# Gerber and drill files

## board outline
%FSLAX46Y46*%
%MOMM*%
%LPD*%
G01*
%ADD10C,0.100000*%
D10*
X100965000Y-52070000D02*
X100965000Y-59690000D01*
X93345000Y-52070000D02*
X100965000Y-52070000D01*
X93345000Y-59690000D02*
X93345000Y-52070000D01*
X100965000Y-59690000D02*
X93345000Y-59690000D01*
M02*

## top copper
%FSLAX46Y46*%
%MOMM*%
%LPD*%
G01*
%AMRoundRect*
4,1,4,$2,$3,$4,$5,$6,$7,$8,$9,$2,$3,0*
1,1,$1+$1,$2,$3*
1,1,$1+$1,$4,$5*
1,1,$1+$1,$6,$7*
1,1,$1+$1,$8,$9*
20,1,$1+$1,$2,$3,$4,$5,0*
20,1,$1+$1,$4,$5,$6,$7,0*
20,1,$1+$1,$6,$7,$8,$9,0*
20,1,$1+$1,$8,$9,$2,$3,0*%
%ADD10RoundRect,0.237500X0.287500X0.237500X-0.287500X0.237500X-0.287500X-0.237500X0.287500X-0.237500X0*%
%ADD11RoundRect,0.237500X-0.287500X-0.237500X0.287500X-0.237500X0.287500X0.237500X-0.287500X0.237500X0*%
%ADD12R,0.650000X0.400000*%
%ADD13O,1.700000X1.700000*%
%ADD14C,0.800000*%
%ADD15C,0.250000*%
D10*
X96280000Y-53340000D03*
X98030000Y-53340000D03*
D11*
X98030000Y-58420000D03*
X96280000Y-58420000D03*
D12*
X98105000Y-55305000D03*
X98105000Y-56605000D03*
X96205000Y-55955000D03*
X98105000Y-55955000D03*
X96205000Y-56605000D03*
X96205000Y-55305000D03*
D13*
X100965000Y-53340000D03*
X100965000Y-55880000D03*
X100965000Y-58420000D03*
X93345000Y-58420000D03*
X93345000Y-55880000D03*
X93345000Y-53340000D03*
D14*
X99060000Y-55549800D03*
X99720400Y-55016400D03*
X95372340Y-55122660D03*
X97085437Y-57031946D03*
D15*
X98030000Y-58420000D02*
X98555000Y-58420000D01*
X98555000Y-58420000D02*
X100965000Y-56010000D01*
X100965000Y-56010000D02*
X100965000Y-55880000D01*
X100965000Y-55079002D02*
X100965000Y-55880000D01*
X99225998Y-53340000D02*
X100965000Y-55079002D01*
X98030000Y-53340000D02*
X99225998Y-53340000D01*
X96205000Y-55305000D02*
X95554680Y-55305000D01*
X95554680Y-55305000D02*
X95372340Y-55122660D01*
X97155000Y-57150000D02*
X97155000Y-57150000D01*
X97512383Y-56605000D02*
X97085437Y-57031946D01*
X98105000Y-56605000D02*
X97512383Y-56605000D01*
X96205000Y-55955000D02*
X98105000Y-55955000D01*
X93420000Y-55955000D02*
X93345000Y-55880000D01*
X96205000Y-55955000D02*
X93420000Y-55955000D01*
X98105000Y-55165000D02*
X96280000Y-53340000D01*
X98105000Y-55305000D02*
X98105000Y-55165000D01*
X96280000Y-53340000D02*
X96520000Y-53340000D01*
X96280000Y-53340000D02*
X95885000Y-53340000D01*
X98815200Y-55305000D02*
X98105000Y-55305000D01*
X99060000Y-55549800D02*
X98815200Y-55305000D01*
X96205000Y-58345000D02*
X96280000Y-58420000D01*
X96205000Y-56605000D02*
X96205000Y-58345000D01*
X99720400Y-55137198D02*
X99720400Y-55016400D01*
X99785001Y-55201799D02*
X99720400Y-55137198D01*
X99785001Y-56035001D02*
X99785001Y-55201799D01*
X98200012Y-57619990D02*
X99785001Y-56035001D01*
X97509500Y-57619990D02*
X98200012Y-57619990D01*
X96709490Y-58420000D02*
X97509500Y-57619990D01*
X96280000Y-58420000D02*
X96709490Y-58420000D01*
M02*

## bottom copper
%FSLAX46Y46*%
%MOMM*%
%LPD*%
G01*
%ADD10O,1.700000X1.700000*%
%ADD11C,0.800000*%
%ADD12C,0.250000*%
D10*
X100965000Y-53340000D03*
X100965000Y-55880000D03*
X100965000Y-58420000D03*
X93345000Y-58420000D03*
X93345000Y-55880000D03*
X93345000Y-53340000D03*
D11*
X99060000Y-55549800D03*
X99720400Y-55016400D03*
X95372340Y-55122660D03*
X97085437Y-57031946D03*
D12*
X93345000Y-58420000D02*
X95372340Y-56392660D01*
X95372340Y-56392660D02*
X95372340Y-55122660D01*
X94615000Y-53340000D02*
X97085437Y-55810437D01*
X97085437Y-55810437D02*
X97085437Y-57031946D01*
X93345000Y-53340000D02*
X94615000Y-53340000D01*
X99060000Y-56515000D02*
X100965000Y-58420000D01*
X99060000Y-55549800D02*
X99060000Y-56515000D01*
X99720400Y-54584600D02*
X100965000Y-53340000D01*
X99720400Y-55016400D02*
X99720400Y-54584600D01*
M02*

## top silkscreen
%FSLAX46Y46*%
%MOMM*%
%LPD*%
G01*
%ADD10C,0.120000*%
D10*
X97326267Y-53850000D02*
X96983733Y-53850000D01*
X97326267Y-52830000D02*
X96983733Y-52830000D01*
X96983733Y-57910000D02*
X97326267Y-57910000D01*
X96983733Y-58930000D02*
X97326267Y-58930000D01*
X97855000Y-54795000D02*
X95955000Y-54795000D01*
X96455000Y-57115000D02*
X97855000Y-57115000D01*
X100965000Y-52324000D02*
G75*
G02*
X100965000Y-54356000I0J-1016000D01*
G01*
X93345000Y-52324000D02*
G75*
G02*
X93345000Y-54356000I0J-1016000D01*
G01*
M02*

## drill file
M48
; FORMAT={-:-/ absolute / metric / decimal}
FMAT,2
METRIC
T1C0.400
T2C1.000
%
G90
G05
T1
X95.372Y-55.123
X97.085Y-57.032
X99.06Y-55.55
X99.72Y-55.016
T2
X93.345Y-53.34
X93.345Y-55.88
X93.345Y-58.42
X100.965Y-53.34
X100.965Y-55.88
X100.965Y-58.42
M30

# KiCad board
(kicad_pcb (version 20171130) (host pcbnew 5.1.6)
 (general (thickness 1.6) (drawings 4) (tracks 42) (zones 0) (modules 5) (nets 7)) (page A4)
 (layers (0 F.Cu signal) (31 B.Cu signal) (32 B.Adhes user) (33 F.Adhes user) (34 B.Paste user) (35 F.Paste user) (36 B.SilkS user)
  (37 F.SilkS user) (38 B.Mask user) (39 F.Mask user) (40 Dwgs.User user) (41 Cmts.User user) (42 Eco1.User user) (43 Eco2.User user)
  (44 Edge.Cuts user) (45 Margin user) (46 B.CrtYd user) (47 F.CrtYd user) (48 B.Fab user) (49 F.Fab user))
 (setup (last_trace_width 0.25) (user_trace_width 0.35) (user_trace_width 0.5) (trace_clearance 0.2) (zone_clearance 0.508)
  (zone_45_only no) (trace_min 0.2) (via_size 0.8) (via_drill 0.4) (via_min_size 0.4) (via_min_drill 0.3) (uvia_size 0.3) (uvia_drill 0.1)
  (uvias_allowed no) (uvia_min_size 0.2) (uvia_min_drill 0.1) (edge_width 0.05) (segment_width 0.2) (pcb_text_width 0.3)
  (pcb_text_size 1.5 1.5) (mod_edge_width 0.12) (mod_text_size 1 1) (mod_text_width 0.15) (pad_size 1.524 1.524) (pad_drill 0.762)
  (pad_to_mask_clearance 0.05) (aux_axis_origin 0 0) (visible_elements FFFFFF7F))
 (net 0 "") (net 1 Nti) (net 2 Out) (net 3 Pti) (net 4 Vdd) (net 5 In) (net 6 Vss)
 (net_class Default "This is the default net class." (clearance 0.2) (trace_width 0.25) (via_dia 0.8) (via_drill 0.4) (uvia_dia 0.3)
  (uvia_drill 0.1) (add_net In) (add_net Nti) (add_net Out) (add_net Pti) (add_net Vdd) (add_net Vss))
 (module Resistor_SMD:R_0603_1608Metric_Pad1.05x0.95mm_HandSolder (layer F.Cu) (at 97.155 53.34 180)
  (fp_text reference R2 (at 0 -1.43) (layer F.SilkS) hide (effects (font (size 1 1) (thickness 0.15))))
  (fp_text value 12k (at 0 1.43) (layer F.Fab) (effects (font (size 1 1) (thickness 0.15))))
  (fp_line (start -0.171267 -0.51) (end 0.171267 -0.51) (layer F.SilkS) (width 0.12))
  (fp_line (start -0.171267 0.51) (end 0.171267 0.51) (layer F.SilkS) (width 0.12))
  (pad 2 smd roundrect (at 0.875 0 180) (size 1.05 0.95) (layers F.Cu F.Paste F.Mask) (roundrect_rratio 0.25) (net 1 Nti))
  (pad 1 smd roundrect (at -0.875 0 180) (size 1.05 0.95) (layers F.Cu F.Paste F.Mask) (roundrect_rratio 0.25) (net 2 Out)))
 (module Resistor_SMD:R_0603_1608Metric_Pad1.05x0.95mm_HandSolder (layer F.Cu) (at 97.155 58.42)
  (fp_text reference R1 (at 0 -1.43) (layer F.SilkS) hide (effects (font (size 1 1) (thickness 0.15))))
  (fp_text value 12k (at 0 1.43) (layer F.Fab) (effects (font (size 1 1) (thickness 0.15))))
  (fp_line (start -0.171267 -0.51) (end 0.171267 -0.51) (layer F.SilkS) (width 0.12))
  (fp_line (start -0.171267 0.51) (end 0.171267 0.51) (layer F.SilkS) (width 0.12))
  (pad 2 smd roundrect (at 0.875 0) (size 1.05 0.95) (layers F.Cu F.Paste F.Mask) (roundrect_rratio 0.25) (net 2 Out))
  (pad 1 smd roundrect (at -0.875 0) (size 1.05 0.95) (layers F.Cu F.Paste F.Mask) (roundrect_rratio 0.25) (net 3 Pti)))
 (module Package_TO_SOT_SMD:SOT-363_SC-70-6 (layer F.Cu) (at 97.155 55.955)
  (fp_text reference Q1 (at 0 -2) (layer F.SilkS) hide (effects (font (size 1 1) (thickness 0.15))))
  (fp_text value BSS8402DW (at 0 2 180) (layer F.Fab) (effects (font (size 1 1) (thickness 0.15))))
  (fp_line (start 0.7 -1.16) (end -1.2 -1.16) (layer F.SilkS) (width 0.12))
  (fp_line (start -0.7 1.16) (end 0.7 1.16) (layer F.SilkS) (width 0.12))
  (pad 6 smd rect (at 0.95 -0.65) (size 0.65 0.4) (layers F.Cu F.Paste F.Mask) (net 1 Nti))
  (pad 4 smd rect (at 0.95 0.65) (size 0.65 0.4) (layers F.Cu F.Paste F.Mask) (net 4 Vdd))
  (pad 2 smd rect (at -0.95 0) (size 0.65 0.4) (layers F.Cu F.Paste F.Mask) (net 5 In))
  (pad 5 smd rect (at 0.95 0) (size 0.65 0.4) (layers F.Cu F.Paste F.Mask) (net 5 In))
  (pad 3 smd rect (at -0.95 0.65) (size 0.65 0.4) (layers F.Cu F.Paste F.Mask) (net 3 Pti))
  (pad 1 smd rect (at -0.95 -0.65) (size 0.65 0.4) (layers F.Cu F.Paste F.Mask) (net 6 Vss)))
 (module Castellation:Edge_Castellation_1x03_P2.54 (layer F.Cu) (at 100.965 53.34)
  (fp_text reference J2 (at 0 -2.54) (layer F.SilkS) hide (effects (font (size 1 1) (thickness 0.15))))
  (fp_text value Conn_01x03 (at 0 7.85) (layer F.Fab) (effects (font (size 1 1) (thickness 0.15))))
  (fp_arc (start 0 0) (end 0 1.016) (angle -180) (layer F.SilkS) (width 0.12))
  (pad 1 thru_hole oval (at 0 0) (size 1.7 1.7) (drill 1) (layers *.Cu *.Mask) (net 3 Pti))
  (pad 2 thru_hole oval (at 0 2.54) (size 1.7 1.7) (drill 1) (layers *.Cu *.Mask) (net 2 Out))
  (pad 3 thru_hole oval (at 0 5.08) (size 1.7 1.7) (drill 1) (layers *.Cu *.Mask) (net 1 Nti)))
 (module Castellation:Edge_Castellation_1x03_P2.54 (layer F.Cu) (at 93.345 53.34)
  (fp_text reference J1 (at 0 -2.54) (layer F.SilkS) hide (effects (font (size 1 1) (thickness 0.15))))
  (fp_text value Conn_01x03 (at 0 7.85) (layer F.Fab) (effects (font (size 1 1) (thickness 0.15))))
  (fp_arc (start 0 0) (end 0 1.016) (angle -180) (layer F.SilkS) (width 0.12))
  (pad 3 thru_hole oval (at 0 5.08) (size 1.7 1.7) (drill 1) (layers *.Cu *.Mask) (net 6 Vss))
  (pad 2 thru_hole oval (at 0 2.54) (size 1.7 1.7) (drill 1) (layers *.Cu *.Mask) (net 5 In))
  (pad 1 thru_hole oval (at 0 0) (size 1.7 1.7) (drill 1) (layers *.Cu *.Mask) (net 4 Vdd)))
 (gr_line (start 100.965 52.07) (end 100.965 59.69) (layer Edge.Cuts) (width 0.1))
 (gr_line (start 93.345 52.07) (end 100.965 52.07) (layer Edge.Cuts) (width 0.1))
 (gr_line (start 93.345 59.69) (end 93.345 52.07) (layer Edge.Cuts) (width 0.1))
 (gr_line (start 100.965 59.69) (end 93.345 59.69) (layer Edge.Cuts) (width 0.1))
 (via (at 99.06 55.5498) (size 0.8) (drill 0.4) (layers F.Cu B.Cu) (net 1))
 (via (at 99.7204 55.0164) (size 0.8) (drill 0.4) (layers F.Cu B.Cu) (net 3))
 (segment (start 98.03 58.42) (end 98.555 58.42) (width 0.25) (layer F.Cu) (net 2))
 (segment (start 98.555 58.42) (end 100.965 56.01) (width 0.25) (layer F.Cu) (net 2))
 (segment (start 100.965 56.01) (end 100.965 55.88) (width 0.25) (layer F.Cu) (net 2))
 (segment (start 100.965 55.079002) (end 100.965 55.88) (width 0.25) (layer F.Cu) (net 2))
 (segment (start 99.225998 53.34) (end 100.965 55.079002) (width 0.25) (layer F.Cu) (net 2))
 (segment (start 98.03 53.34) (end 99.225998 53.34) (width 0.25) (layer F.Cu) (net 2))
 (segment (start 96.205 55.305) (end 95.55468 55.305) (width 0.25) (layer F.Cu) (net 6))
 (segment (start 93.345 58.42) (end 95.37234 56.39266) (width 0.25) (layer B.Cu) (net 6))
 (segment (start 95.55468 55.305) (end 95.37234 55.12266) (width 0.25) (layer F.Cu) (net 6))
 (segment (start 95.37234 56.39266) (end 95.37234 55.12266) (width 0.25) (layer B.Cu) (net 6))
 (via (at 95.37234 55.12266) (size 0.8) (drill 0.4) (layers F.Cu B.Cu) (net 6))
 (segment (start 97.155 57.15) (end 97.155 57.15) (width 0.25) (layer F.Cu) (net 4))
 (segment (start 94.615 53.34) (end 97.085437 55.810437) (width 0.25) (layer B.Cu) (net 4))
 (segment (start 97.512383 56.605) (end 97.085437 57.031946) (width 0.25) (layer F.Cu) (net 4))
 (via (at 97.085437 57.031946) (size 0.8) (drill 0.4) (layers F.Cu B.Cu) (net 4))
 (segment (start 98.105 56.605) (end 97.512383 56.605) (width 0.25) (layer F.Cu) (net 4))
 (segment (start 97.085437 55.810437) (end 97.085437 57.031946) (width 0.25) (layer B.Cu) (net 4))
 (segment (start 93.345 53.34) (end 94.615 53.34) (width 0.25) (layer B.Cu) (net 4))
 (segment (start 96.205 55.955) (end 98.105 55.955) (width 0.25) (layer F.Cu) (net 5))
 (segment (start 93.42 55.955) (end 93.345 55.88) (width 0.25) (layer F.Cu) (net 5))
 (segment (start 96.205 55.955) (end 93.42 55.955) (width 0.25) (layer F.Cu) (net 5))
 (segment (start 98.105 55.165) (end 96.28 53.34) (width 0.25) (layer F.Cu) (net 1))
 (segment (start 98.105 55.305) (end 98.105 55.165) (width 0.25) (layer F.Cu) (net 1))
 (segment (start 96.28 53.34) (end 96.52 53.34) (width 0.25) (layer F.Cu) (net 1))
 (segment (start 96.28 53.34) (end 95.885 53.34) (width 0.25) (layer F.Cu) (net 1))
 (segment (start 98.8152 55.305) (end 98.105 55.305) (width 0.25) (layer F.Cu) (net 1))
 (segment (start 99.06 55.5498) (end 98.8152 55.305) (width 0.25) (layer F.Cu) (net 1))
 (segment (start 99.06 56.515) (end 100.965 58.42) (width 0.25) (layer B.Cu) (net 1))
 (segment (start 99.06 55.5498) (end 99.06 56.515) (width 0.25) (layer B.Cu) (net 1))
 (segment (start 96.205 58.345) (end 96.28 58.42) (width 0.25) (layer F.Cu) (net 3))
 (segment (start 96.205 56.605) (end 96.205 58.345) (width 0.25) (layer F.Cu) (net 3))
 (segment (start 99.7204 55.137198) (end 99.7204 55.0164) (width 0.25) (layer F.Cu) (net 3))
 (segment (start 99.785001 55.201799) (end 99.7204 55.137198) (width 0.25) (layer F.Cu) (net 3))
 (segment (start 99.785001 56.035001) (end 99.785001 55.201799) (width 0.25) (layer F.Cu) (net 3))
 (segment (start 98.200012 57.61999) (end 99.785001 56.035001) (width 0.25) (layer F.Cu) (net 3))
 (segment (start 97.5095 57.61999) (end 98.200012 57.61999) (width 0.25) (layer F.Cu) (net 3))
 (segment (start 96.70949 58.42) (end 97.5095 57.61999) (width 0.25) (layer F.Cu) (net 3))
 (segment (start 96.28 58.42) (end 96.70949 58.42) (width 0.25) (layer F.Cu) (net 3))
 (segment (start 99.7204 54.5846) (end 100.965 53.34) (width 0.25) (layer B.Cu) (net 3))
 (segment (start 99.7204 55.0164) (end 99.7204 54.5846) (width 0.25) (layer B.Cu) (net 3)))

